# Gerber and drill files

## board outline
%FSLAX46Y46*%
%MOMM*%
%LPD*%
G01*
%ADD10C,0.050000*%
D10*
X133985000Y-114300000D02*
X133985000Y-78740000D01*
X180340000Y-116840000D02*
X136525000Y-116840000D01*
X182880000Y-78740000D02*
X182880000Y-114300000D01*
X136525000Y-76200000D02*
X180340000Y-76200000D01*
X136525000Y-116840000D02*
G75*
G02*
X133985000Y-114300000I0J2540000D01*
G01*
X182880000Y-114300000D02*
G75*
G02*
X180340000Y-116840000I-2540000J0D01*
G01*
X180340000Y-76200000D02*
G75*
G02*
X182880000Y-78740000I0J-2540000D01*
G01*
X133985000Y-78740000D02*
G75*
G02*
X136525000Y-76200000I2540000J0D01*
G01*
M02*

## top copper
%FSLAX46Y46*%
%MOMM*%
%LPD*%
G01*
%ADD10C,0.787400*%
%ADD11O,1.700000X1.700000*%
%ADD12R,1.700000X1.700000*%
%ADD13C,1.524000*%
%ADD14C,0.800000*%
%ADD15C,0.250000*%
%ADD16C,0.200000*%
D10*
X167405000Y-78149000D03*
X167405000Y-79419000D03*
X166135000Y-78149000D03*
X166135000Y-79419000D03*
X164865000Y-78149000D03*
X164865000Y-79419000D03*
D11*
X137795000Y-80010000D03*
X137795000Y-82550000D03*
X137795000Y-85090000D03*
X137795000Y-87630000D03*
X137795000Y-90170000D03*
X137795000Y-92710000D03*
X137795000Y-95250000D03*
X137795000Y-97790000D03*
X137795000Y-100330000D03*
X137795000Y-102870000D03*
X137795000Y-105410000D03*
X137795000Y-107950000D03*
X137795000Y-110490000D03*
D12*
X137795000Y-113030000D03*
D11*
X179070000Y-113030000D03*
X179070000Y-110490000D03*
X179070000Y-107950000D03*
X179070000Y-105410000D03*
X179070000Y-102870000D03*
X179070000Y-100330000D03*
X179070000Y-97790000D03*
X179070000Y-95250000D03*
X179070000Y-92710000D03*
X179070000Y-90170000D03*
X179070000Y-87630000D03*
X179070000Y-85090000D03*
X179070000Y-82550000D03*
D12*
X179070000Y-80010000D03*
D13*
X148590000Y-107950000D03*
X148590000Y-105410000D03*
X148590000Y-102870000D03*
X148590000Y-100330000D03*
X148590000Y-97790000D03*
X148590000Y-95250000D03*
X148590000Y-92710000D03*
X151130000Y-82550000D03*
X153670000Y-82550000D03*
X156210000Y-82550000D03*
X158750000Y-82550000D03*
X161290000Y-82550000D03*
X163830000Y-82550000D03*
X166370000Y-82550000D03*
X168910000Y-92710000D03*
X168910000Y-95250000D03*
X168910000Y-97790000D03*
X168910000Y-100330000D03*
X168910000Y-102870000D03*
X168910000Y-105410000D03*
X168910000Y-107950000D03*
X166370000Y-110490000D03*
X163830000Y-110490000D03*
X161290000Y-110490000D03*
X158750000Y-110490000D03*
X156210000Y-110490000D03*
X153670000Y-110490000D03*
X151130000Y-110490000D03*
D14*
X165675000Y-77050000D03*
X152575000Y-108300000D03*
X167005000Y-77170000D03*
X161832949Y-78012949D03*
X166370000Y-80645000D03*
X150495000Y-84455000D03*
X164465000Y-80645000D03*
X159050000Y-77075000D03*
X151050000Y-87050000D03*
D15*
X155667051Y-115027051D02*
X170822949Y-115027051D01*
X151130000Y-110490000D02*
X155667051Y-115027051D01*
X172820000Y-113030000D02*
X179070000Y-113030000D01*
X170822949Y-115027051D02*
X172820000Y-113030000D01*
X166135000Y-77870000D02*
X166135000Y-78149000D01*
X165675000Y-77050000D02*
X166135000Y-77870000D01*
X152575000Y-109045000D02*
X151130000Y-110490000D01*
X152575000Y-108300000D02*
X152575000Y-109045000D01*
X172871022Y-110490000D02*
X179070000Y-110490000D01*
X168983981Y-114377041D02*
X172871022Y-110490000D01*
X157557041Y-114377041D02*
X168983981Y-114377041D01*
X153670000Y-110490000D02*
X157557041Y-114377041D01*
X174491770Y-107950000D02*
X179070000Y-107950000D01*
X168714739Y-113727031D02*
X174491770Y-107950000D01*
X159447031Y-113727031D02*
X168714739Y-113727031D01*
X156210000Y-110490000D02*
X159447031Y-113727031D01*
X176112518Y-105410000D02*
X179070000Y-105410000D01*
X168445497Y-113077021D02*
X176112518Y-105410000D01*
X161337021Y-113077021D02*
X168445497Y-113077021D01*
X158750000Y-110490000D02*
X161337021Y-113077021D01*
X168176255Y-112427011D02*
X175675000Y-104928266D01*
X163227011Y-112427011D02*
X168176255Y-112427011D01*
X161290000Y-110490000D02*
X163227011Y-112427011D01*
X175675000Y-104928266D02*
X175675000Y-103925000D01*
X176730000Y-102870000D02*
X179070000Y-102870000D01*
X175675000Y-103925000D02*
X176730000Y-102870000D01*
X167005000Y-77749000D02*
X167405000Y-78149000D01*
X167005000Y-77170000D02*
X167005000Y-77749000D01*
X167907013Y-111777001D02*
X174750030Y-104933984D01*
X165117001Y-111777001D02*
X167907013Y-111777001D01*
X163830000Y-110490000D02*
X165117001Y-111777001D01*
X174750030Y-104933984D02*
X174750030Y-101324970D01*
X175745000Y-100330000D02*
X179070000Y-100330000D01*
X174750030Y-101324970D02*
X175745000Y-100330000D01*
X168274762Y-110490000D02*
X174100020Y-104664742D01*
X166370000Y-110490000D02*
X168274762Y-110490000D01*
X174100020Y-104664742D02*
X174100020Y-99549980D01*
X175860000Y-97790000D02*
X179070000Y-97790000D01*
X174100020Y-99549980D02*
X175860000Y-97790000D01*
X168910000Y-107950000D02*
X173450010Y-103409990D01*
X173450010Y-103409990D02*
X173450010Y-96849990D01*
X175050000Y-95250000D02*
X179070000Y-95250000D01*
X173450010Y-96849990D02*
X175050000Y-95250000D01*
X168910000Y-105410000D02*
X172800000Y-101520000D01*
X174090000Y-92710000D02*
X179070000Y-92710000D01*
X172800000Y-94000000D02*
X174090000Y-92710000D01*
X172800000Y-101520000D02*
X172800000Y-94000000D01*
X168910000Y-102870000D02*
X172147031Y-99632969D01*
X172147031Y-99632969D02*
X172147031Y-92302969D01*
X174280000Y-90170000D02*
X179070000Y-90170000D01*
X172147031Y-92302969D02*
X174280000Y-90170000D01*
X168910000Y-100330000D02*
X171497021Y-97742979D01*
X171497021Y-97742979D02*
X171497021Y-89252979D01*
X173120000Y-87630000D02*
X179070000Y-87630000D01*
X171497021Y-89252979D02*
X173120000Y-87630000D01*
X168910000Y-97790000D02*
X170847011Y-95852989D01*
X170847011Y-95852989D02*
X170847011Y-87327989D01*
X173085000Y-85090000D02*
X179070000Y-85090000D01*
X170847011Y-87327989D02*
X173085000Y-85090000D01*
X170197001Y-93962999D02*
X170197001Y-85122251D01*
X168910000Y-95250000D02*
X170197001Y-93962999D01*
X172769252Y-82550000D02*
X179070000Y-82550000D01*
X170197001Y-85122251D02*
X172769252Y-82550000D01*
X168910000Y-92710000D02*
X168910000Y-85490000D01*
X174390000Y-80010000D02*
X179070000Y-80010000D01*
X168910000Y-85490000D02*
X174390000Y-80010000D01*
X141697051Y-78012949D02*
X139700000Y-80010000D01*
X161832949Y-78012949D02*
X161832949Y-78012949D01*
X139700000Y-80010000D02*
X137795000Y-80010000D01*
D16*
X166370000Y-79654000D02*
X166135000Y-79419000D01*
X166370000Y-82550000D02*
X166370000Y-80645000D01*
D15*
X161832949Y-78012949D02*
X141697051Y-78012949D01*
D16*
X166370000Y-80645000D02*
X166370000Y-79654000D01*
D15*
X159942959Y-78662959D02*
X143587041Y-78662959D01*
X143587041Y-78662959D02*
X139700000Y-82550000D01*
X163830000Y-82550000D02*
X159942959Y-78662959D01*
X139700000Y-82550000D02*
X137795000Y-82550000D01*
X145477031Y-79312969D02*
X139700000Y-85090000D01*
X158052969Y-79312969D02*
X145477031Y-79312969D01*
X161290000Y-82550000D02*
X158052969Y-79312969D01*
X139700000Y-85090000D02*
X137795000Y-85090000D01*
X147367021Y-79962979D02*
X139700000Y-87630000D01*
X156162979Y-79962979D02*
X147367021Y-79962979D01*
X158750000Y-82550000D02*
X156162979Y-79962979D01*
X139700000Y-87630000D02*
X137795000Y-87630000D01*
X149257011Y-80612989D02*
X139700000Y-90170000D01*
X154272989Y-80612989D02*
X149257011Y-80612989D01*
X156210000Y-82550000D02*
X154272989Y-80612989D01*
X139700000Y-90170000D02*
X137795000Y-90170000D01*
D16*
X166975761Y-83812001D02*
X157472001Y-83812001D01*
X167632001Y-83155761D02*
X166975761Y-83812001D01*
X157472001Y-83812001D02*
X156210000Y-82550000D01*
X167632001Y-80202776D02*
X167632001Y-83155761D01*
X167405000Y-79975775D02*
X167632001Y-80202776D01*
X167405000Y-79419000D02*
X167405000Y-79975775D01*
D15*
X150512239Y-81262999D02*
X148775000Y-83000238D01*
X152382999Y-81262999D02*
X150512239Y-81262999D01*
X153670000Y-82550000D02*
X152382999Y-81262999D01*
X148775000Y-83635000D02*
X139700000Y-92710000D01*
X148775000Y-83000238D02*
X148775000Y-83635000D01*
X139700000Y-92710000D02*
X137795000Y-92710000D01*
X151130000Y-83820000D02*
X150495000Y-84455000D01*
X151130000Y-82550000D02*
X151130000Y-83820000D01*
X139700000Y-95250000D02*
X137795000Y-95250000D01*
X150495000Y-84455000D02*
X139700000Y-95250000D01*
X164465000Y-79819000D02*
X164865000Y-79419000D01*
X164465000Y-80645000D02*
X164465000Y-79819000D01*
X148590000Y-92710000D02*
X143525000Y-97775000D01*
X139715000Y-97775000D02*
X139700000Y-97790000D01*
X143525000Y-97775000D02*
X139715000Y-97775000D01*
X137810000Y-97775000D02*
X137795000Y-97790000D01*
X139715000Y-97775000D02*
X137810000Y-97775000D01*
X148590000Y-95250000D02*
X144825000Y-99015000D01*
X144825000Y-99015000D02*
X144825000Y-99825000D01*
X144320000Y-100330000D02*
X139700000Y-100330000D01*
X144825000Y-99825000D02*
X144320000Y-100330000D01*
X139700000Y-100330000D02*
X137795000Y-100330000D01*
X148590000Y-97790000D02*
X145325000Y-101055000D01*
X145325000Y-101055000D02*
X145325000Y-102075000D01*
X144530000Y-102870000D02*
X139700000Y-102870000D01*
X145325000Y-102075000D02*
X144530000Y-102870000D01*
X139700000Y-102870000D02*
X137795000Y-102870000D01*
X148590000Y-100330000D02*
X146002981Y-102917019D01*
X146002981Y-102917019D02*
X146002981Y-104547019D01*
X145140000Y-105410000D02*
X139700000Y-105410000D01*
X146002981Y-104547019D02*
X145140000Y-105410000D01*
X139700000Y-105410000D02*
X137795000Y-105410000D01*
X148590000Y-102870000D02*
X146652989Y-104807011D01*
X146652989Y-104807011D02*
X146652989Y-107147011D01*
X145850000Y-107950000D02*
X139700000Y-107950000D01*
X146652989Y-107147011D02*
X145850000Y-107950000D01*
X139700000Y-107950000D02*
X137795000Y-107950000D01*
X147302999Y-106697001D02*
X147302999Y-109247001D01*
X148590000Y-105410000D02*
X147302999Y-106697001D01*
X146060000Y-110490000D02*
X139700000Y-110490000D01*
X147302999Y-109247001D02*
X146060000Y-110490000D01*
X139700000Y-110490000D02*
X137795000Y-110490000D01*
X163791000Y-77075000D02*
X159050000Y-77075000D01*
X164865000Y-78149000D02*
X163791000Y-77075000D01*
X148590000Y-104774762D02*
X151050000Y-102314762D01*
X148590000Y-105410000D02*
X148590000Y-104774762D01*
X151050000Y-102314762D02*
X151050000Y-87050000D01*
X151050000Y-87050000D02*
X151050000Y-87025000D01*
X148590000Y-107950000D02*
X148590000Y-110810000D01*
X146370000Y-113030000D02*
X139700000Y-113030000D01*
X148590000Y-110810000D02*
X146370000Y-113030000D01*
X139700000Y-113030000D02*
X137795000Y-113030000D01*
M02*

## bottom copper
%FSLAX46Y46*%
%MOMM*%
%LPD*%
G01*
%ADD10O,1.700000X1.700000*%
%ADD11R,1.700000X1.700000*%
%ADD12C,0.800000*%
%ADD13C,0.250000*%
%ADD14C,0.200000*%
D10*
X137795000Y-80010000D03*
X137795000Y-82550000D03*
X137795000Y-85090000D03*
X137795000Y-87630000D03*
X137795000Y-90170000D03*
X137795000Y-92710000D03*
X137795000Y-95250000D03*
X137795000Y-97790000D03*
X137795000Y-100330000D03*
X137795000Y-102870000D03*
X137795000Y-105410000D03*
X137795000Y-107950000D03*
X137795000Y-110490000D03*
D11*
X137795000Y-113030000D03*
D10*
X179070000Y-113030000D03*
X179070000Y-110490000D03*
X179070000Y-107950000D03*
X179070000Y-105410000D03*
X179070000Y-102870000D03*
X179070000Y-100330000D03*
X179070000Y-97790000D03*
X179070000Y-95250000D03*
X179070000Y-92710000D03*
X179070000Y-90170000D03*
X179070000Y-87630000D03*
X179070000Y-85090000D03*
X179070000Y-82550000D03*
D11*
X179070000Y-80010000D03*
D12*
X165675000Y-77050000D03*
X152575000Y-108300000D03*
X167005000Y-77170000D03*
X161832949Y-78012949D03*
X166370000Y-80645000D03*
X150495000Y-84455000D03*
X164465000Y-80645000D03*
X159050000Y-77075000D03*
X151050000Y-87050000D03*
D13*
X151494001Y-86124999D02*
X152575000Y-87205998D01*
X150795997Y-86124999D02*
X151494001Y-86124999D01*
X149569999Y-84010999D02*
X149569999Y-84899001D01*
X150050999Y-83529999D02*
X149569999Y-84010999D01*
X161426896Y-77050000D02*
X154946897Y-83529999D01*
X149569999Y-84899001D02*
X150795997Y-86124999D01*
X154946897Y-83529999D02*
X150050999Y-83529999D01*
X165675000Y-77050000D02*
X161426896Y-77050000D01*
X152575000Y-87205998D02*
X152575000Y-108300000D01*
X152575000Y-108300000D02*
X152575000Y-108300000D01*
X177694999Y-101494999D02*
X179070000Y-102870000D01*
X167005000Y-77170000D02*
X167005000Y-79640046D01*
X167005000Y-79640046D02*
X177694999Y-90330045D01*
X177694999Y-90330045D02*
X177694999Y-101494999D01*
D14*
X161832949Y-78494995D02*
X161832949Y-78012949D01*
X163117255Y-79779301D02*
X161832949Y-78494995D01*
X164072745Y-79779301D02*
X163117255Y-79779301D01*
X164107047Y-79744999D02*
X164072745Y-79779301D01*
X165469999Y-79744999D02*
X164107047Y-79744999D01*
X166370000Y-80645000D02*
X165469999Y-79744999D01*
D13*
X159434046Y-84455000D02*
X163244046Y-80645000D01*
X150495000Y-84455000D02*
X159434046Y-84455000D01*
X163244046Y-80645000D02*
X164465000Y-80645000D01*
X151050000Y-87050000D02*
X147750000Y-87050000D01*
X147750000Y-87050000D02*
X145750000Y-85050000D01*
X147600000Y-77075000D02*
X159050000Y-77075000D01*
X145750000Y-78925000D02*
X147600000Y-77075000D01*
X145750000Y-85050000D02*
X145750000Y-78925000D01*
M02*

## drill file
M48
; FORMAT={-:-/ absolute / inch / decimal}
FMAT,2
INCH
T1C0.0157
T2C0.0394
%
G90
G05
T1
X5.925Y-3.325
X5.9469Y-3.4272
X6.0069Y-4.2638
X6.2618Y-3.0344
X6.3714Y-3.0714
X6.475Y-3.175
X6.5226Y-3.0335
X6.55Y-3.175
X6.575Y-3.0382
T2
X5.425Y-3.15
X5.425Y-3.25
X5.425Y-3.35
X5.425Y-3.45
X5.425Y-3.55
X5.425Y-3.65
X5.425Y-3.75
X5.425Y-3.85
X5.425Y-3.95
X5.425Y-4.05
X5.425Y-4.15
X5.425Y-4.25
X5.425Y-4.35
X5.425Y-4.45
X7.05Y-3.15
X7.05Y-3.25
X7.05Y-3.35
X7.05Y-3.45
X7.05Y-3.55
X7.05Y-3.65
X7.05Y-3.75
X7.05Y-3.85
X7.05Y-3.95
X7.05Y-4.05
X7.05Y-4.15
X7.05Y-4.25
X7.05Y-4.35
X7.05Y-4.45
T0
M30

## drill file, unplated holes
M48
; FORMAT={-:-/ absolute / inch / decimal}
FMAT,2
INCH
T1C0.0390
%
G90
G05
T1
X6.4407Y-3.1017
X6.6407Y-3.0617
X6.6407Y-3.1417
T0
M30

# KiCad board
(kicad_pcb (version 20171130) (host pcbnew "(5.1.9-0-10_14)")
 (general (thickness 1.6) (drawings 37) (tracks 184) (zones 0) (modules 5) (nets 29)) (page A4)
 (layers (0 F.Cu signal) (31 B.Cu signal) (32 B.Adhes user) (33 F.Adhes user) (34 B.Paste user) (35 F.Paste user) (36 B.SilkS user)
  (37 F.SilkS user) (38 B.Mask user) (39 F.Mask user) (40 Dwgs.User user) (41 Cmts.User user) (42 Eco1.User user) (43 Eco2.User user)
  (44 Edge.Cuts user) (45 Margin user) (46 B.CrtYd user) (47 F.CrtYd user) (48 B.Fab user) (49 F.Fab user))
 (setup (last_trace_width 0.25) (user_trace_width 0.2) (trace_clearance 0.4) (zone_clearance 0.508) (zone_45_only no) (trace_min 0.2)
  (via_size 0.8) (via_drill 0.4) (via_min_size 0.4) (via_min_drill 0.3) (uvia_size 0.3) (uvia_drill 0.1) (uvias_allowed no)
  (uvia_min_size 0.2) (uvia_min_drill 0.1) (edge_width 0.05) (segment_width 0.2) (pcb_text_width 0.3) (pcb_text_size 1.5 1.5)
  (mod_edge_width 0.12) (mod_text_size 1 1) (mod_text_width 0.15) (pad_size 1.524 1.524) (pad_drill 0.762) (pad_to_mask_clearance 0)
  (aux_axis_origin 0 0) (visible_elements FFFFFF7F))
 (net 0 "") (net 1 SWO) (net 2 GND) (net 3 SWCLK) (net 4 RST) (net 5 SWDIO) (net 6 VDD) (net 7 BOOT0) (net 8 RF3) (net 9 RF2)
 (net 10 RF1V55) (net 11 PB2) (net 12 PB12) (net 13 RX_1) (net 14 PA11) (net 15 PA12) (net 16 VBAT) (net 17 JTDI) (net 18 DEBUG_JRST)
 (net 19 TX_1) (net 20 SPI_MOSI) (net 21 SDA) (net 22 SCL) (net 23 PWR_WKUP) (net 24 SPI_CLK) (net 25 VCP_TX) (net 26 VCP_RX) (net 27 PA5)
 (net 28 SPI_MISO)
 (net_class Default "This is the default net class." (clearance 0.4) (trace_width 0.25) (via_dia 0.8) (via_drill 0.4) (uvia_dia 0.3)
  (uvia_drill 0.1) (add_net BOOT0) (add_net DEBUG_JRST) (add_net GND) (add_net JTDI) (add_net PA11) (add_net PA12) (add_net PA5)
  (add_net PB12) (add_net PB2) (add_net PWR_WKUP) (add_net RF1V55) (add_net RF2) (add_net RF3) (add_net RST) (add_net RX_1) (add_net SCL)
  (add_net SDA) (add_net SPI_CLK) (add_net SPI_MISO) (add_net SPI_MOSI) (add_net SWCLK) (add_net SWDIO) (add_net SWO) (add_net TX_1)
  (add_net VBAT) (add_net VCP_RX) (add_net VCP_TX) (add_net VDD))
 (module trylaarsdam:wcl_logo (layer F.Cu) (at 148 114.25)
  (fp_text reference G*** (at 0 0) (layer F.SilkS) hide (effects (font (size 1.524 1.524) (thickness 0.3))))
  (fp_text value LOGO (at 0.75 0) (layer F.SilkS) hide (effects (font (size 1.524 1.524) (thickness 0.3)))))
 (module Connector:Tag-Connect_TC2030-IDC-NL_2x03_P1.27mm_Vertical (layer F.Cu) (at 166.135 78.784)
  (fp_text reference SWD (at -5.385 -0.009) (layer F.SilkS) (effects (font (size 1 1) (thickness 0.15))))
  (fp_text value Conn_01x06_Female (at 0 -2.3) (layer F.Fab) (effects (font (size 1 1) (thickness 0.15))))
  (pad 6 connect circle (at 1.27 -0.635) (size 0.7874 0.7874) (layers F.Cu F.Mask) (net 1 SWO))
  (pad 5 connect circle (at 1.27 0.635) (size 0.7874 0.7874) (layers F.Cu F.Mask) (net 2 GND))
  (pad 4 connect circle (at 0 -0.635) (size 0.7874 0.7874) (layers F.Cu F.Mask) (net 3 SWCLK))
  (pad 3 connect circle (at 0 0.635) (size 0.7874 0.7874) (layers F.Cu F.Mask) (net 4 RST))
  (pad 2 connect circle (at -1.27 -0.635) (size 0.7874 0.7874) (layers F.Cu F.Mask) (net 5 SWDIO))
  (pad 1 connect circle (at -1.27 0.635) (size 0.7874 0.7874) (layers F.Cu F.Mask) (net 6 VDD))
  (pad "" np_thru_hole circle (at -2.54 0) (size 0.9906 0.9906) (drill 0.9906) (layers *.Cu *.Mask))
  (pad "" np_thru_hole circle (at 2.54 1.016) (size 0.9906 0.9906) (drill 0.9906) (layers *.Cu *.Mask))
  (pad "" np_thru_hole circle (at 2.54 -1.016) (size 0.9906 0.9906) (drill 0.9906) (layers *.Cu *.Mask)))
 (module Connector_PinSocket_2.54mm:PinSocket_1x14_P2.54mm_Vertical (layer F.Cu) (at 137.795 113.03 180)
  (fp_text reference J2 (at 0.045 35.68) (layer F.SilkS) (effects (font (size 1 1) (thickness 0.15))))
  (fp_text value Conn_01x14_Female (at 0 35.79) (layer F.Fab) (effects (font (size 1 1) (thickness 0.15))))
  (pad 14 thru_hole oval (at 0 33.02 180) (size 1.7 1.7) (drill 1) (layers *.Cu *.Mask) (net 4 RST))
  (pad 13 thru_hole oval (at 0 30.48 180) (size 1.7 1.7) (drill 1) (layers *.Cu *.Mask) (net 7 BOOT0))
  (pad 12 thru_hole oval (at 0 27.94 180) (size 1.7 1.7) (drill 1) (layers *.Cu *.Mask) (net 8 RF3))
  (pad 11 thru_hole oval (at 0 25.4 180) (size 1.7 1.7) (drill 1) (layers *.Cu *.Mask) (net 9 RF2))
  (pad 10 thru_hole oval (at 0 22.86 180) (size 1.7 1.7) (drill 1) (layers *.Cu *.Mask) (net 2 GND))
  (pad 9 thru_hole oval (at 0 20.32 180) (size 1.7 1.7) (drill 1) (layers *.Cu *.Mask) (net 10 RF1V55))
  (pad 8 thru_hole oval (at 0 17.78 180) (size 1.7 1.7) (drill 1) (layers *.Cu *.Mask) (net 6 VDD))
  (pad 7 thru_hole oval (at 0 15.24 180) (size 1.7 1.7) (drill 1) (layers *.Cu *.Mask) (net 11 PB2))
  (pad 6 thru_hole oval (at 0 12.7 180) (size 1.7 1.7) (drill 1) (layers *.Cu *.Mask) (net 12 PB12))
  (pad 5 thru_hole oval (at 0 10.16 180) (size 1.7 1.7) (drill 1) (layers *.Cu *.Mask) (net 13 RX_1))
  (pad 4 thru_hole oval (at 0 7.62 180) (size 1.7 1.7) (drill 1) (layers *.Cu *.Mask) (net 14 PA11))
  (pad 3 thru_hole oval (at 0 5.08 180) (size 1.7 1.7) (drill 1) (layers *.Cu *.Mask) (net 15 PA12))
  (pad 2 thru_hole oval (at 0 2.54 180) (size 1.7 1.7) (drill 1) (layers *.Cu *.Mask) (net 5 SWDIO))
  (pad 1 thru_hole rect (at 0 0 180) (size 1.7 1.7) (drill 1) (layers *.Cu *.Mask) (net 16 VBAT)))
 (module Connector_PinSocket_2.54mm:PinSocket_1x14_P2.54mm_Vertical (layer F.Cu) (at 179.07 80.01)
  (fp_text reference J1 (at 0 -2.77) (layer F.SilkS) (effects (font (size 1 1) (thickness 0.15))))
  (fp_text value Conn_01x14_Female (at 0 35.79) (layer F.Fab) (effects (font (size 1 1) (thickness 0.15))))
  (pad 14 thru_hole oval (at 0 33.02) (size 1.7 1.7) (drill 1) (layers *.Cu *.Mask) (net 3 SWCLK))
  (pad 13 thru_hole oval (at 0 30.48) (size 1.7 1.7) (drill 1) (layers *.Cu *.Mask) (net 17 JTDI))
  (pad 12 thru_hole oval (at 0 27.94) (size 1.7 1.7) (drill 1) (layers *.Cu *.Mask) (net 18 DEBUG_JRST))
  (pad 11 thru_hole oval (at 0 25.4) (size 1.7 1.7) (drill 1) (layers *.Cu *.Mask) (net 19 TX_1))
  (pad 10 thru_hole oval (at 0 22.86) (size 1.7 1.7) (drill 1) (layers *.Cu *.Mask) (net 1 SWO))
  (pad 9 thru_hole oval (at 0 20.32) (size 1.7 1.7) (drill 1) (layers *.Cu *.Mask) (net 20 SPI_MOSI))
  (pad 8 thru_hole oval (at 0 17.78) (size 1.7 1.7) (drill 1) (layers *.Cu *.Mask) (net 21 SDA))
  (pad 7 thru_hole oval (at 0 15.24) (size 1.7 1.7) (drill 1) (layers *.Cu *.Mask) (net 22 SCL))
  (pad 6 thru_hole oval (at 0 12.7) (size 1.7 1.7) (drill 1) (layers *.Cu *.Mask) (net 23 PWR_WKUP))
  (pad 5 thru_hole oval (at 0 10.16) (size 1.7 1.7) (drill 1) (layers *.Cu *.Mask) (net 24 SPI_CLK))
  (pad 4 thru_hole oval (at 0 7.62) (size 1.7 1.7) (drill 1) (layers *.Cu *.Mask) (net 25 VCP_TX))
  (pad 3 thru_hole oval (at 0 5.08) (size 1.7 1.7) (drill 1) (layers *.Cu *.Mask) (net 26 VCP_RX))
  (pad 2 thru_hole oval (at 0 2.54) (size 1.7 1.7) (drill 1) (layers *.Cu *.Mask) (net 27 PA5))
  (pad 1 thru_hole rect (at 0 0) (size 1.7 1.7) (drill 1) (layers *.Cu *.Mask) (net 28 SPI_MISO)))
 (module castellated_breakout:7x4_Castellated (layer F.Cu) (at 163.83 97.79 90)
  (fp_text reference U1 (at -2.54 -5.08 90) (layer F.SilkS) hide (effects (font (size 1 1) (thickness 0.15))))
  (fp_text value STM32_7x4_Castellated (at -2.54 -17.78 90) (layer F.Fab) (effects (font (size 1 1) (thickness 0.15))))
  (pad 28 smd circle (at -10.16 -15.24 90) (size 1.524 1.524) (layers F.Cu F.Paste F.Mask) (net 16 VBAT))
  (pad 27 smd circle (at -7.62 -15.24 90) (size 1.524 1.524) (layers F.Cu F.Paste F.Mask) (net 5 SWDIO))
  (pad 26 smd circle (at -5.08 -15.24 90) (size 1.524 1.524) (layers F.Cu F.Paste F.Mask) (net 15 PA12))
  (pad 25 smd circle (at -2.54 -15.24 90) (size 1.524 1.524) (layers F.Cu F.Paste F.Mask) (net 14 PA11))
  (pad 24 smd circle (at 0 -15.24 90) (size 1.524 1.524) (layers F.Cu F.Paste F.Mask) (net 13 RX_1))
  (pad 23 smd circle (at 2.54 -15.24 90) (size 1.524 1.524) (layers F.Cu F.Paste F.Mask) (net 12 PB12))
  (pad 22 smd circle (at 5.08 -15.24 90) (size 1.524 1.524) (layers F.Cu F.Paste F.Mask) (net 11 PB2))
  (pad 21 smd circle (at 15.24 -12.7 90) (size 1.524 1.524) (layers F.Cu F.Paste F.Mask) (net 6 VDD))
  (pad 20 smd circle (at 15.24 -10.16 90) (size 1.524 1.524) (layers F.Cu F.Paste F.Mask) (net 10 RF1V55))
  (pad 19 smd circle (at 15.24 -7.62 90) (size 1.524 1.524) (layers F.Cu F.Paste F.Mask) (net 2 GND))
  (pad 18 smd circle (at 15.24 -5.08 90) (size 1.524 1.524) (layers F.Cu F.Paste F.Mask) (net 9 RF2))
  (pad 17 smd circle (at 15.24 -2.54 90) (size 1.524 1.524) (layers F.Cu F.Paste F.Mask) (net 8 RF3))
  (pad 16 smd circle (at 15.24 0 90) (size 1.524 1.524) (layers F.Cu F.Paste F.Mask) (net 7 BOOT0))
  (pad 15 smd circle (at 15.24 2.54 90) (size 1.524 1.524) (layers F.Cu F.Paste F.Mask) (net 4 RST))
  (pad 14 smd circle (at 5.08 5.08 90) (size 1.524 1.524) (layers F.Cu F.Paste F.Mask) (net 28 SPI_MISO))
  (pad 13 smd circle (at 2.54 5.08 90) (size 1.524 1.524) (layers F.Cu F.Paste F.Mask) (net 27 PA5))
  (pad 12 smd circle (at 0 5.08 90) (size 1.524 1.524) (layers F.Cu F.Paste F.Mask) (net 26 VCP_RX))
  (pad 11 smd circle (at -2.54 5.08 90) (size 1.524 1.524) (layers F.Cu F.Paste F.Mask) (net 25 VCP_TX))
  (pad 10 smd circle (at -5.08 5.08 90) (size 1.524 1.524) (layers F.Cu F.Paste F.Mask) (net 24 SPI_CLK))
  (pad 9 smd circle (at -7.62 5.08 90) (size 1.524 1.524) (layers F.Cu F.Paste F.Mask) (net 23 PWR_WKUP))
  (pad 8 smd circle (at -10.16 5.08 90) (size 1.524 1.524) (layers F.Cu F.Paste F.Mask) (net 22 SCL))
  (pad 7 smd circle (at -12.7 2.54 90) (size 1.524 1.524) (layers F.Cu F.Paste F.Mask) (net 21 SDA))
  (pad 6 smd circle (at -12.7 0 90) (size 1.524 1.524) (layers F.Cu F.Paste F.Mask) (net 20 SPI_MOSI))
  (pad 5 smd circle (at -12.7 -2.54 90) (size 1.524 1.524) (layers F.Cu F.Paste F.Mask) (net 1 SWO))
  (pad 4 smd circle (at -12.7 -5.08 90) (size 1.524 1.524) (layers F.Cu F.Paste F.Mask) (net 19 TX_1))
  (pad 3 smd circle (at -12.7 -7.62 90) (size 1.524 1.524) (layers F.Cu F.Paste F.Mask) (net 18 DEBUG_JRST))
  (pad 2 smd circle (at -12.7 -10.16 90) (size 1.524 1.524) (layers F.Cu F.Paste F.Mask) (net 17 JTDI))
  (pad 1 smd circle (at -12.7 -12.7 90) (size 1.524 1.524) (layers F.Cu F.Paste F.Mask) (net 3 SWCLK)))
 (gr_line (start 133.985 114.3) (end 133.985 78.74) (layer Edge.Cuts) (width 0.05))
 (gr_line (start 180.34 116.84) (end 136.525 116.84) (layer Edge.Cuts) (width 0.05))
 (gr_line (start 182.88 78.74) (end 182.88 114.3) (layer Edge.Cuts) (width 0.05))
 (gr_line (start 136.525 76.2) (end 180.34 76.2) (layer Edge.Cuts) (width 0.05))
 (gr_arc (start 136.525 114.3) (end 133.985 114.3) (angle -90) (layer Edge.Cuts) (width 0.05))
 (gr_arc (start 180.34 114.3) (end 180.34 116.84) (angle -90) (layer Edge.Cuts) (width 0.05))
 (gr_arc (start 180.34 78.74) (end 182.88 78.74) (angle -90) (layer Edge.Cuts) (width 0.05))
 (gr_arc (start 136.525 78.74) (end 136.525 76.2) (angle -90) (layer Edge.Cuts) (width 0.05))
 (segment (start 155.667051 115.027051) (end 170.822949 115.027051) (width 0.25) (layer F.Cu) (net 3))
 (segment (start 151.13 110.49) (end 155.667051 115.027051) (width 0.25) (layer F.Cu) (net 3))
 (segment (start 172.82 113.03) (end 179.07 113.03) (width 0.25) (layer F.Cu) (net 3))
 (segment (start 170.822949 115.027051) (end 172.82 113.03) (width 0.25) (layer F.Cu) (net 3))
 (segment (start 166.135 77.87) (end 166.135 78.149) (width 0.25) (layer F.Cu) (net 3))
 (segment (start 165.675 77.05) (end 166.135 77.87) (width 0.25) (layer F.Cu) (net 3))
 (via (at 165.675 77.05) (size 0.8) (drill 0.4) (layers F.Cu B.Cu) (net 3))
 (segment (start 151.494001 86.124999) (end 152.575 87.205998) (width 0.25) (layer B.Cu) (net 3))
 (segment (start 150.795997 86.124999) (end 151.494001 86.124999) (width 0.25) (layer B.Cu) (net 3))
 (segment (start 149.569999 84.010999) (end 149.569999 84.899001) (width 0.25) (layer B.Cu) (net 3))
 (segment (start 150.050999 83.529999) (end 149.569999 84.010999) (width 0.25) (layer B.Cu) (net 3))
 (segment (start 161.426896 77.05) (end 154.946897 83.529999) (width 0.25) (layer B.Cu) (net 3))
 (segment (start 149.569999 84.899001) (end 150.795997 86.124999) (width 0.25) (layer B.Cu) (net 3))
 (segment (start 154.946897 83.529999) (end 150.050999 83.529999) (width 0.25) (layer B.Cu) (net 3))
 (segment (start 165.675 77.05) (end 161.426896 77.05) (width 0.25) (layer B.Cu) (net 3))
 (segment (start 152.575 87.205998) (end 152.575 108.3) (width 0.25) (layer B.Cu) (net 3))
 (segment (start 152.575 108.3) (end 152.575 108.3) (width 0.25) (layer B.Cu) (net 3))
 (via (at 152.575 108.3) (size 0.8) (drill 0.4) (layers F.Cu B.Cu) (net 3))
 (segment (start 152.575 109.045) (end 151.13 110.49) (width 0.25) (layer F.Cu) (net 3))
 (segment (start 152.575 108.3) (end 152.575 109.045) (width 0.25) (layer F.Cu) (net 3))
 (segment (start 172.871022 110.49) (end 179.07 110.49) (width 0.25) (layer F.Cu) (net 17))
 (segment (start 168.983981 114.377041) (end 172.871022 110.49) (width 0.25) (layer F.Cu) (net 17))
 (segment (start 157.557041 114.377041) (end 168.983981 114.377041) (width 0.25) (layer F.Cu) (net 17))
 (segment (start 153.67 110.49) (end 157.557041 114.377041) (width 0.25) (layer F.Cu) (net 17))
 (segment (start 174.49177 107.95) (end 179.07 107.95) (width 0.25) (layer F.Cu) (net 18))
 (segment (start 168.714739 113.727031) (end 174.49177 107.95) (width 0.25) (layer F.Cu) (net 18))
 (segment (start 159.447031 113.727031) (end 168.714739 113.727031) (width 0.25) (layer F.Cu) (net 18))
 (segment (start 156.21 110.49) (end 159.447031 113.727031) (width 0.25) (layer F.Cu) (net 18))
 (segment (start 176.112518 105.41) (end 179.07 105.41) (width 0.25) (layer F.Cu) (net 19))
 (segment (start 168.445497 113.077021) (end 176.112518 105.41) (width 0.25) (layer F.Cu) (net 19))
 (segment (start 161.337021 113.077021) (end 168.445497 113.077021) (width 0.25) (layer F.Cu) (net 19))
 (segment (start 158.75 110.49) (end 161.337021 113.077021) (width 0.25) (layer F.Cu) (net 19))
 (segment (start 168.176255 112.427011) (end 175.675 104.928266) (width 0.25) (layer F.Cu) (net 1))
 (segment (start 163.227011 112.427011) (end 168.176255 112.427011) (width 0.25) (layer F.Cu) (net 1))
 (segment (start 161.29 110.49) (end 163.227011 112.427011) (width 0.25) (layer F.Cu) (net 1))
 (segment (start 175.675 104.928266) (end 175.675 103.925) (width 0.25) (layer F.Cu) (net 1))
 (segment (start 176.73 102.87) (end 179.07 102.87) (width 0.25) (layer F.Cu) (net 1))
 (segment (start 175.675 103.925) (end 176.73 102.87) (width 0.25) (layer F.Cu) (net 1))
 (segment (start 177.694999 101.494999) (end 179.07 102.87) (width 0.25) (layer B.Cu) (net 1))
 (segment (start 167.005 77.17) (end 167.005 79.640046) (width 0.25) (layer B.Cu) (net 1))
 (segment (start 167.005 77.749) (end 167.405 78.149) (width 0.25) (layer F.Cu) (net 1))
 (segment (start 167.005 79.640046) (end 177.694999 90.330045) (width 0.25) (layer B.Cu) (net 1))
 (segment (start 177.694999 90.330045) (end 177.694999 101.494999) (width 0.25) (layer B.Cu) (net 1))
 (segment (start 167.005 77.17) (end 167.005 77.749) (width 0.25) (layer F.Cu) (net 1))
 (via (at 167.005 77.17) (size 0.8) (drill 0.4) (layers F.Cu B.Cu) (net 1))
 (segment (start 167.907013 111.777001) (end 174.75003 104.933984) (width 0.25) (layer F.Cu) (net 20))
 (segment (start 165.117001 111.777001) (end 167.907013 111.777001) (width 0.25) (layer F.Cu) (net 20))
 (segment (start 163.83 110.49) (end 165.117001 111.777001) (width 0.25) (layer F.Cu) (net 20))
 (segment (start 174.75003 104.933984) (end 174.75003 101.32497) (width 0.25) (layer F.Cu) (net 20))
 (segment (start 175.745 100.33) (end 179.07 100.33) (width 0.25) (layer F.Cu) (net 20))
 (segment (start 174.75003 101.32497) (end 175.745 100.33) (width 0.25) (layer F.Cu) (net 20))
 (segment (start 168.274762 110.49) (end 174.10002 104.664742) (width 0.25) (layer F.Cu) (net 21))
 (segment (start 166.37 110.49) (end 168.274762 110.49) (width 0.25) (layer F.Cu) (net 21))
 (segment (start 174.10002 104.664742) (end 174.10002 99.54998) (width 0.25) (layer F.Cu) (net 21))
 (segment (start 175.86 97.79) (end 179.07 97.79) (width 0.25) (layer F.Cu) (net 21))
 (segment (start 174.10002 99.54998) (end 175.86 97.79) (width 0.25) (layer F.Cu) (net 21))
 (segment (start 168.91 107.95) (end 173.45001 103.40999) (width 0.25) (layer F.Cu) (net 22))
 (segment (start 173.45001 103.40999) (end 173.45001 96.84999) (width 0.25) (layer F.Cu) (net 22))
 (segment (start 175.05 95.25) (end 179.07 95.25) (width 0.25) (layer F.Cu) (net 22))
 (segment (start 173.45001 96.84999) (end 175.05 95.25) (width 0.25) (layer F.Cu) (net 22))
 (segment (start 168.91 105.41) (end 172.8 101.52) (width 0.25) (layer F.Cu) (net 23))
 (segment (start 174.09 92.71) (end 179.07 92.71) (width 0.25) (layer F.Cu) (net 23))
 (segment (start 172.8 94) (end 174.09 92.71) (width 0.25) (layer F.Cu) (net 23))
 (segment (start 172.8 101.52) (end 172.8 94) (width 0.25) (layer F.Cu) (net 23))
 (segment (start 168.91 102.87) (end 172.147031 99.632969) (width 0.25) (layer F.Cu) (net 24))
 (segment (start 172.147031 99.632969) (end 172.147031 92.302969) (width 0.25) (layer F.Cu) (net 24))
 (segment (start 174.28 90.17) (end 179.07 90.17) (width 0.25) (layer F.Cu) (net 24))
 (segment (start 172.147031 92.302969) (end 174.28 90.17) (width 0.25) (layer F.Cu) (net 24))
 (segment (start 168.91 100.33) (end 171.497021 97.742979) (width 0.25) (layer F.Cu) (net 25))
 (segment (start 171.497021 97.742979) (end 171.497021 89.252979) (width 0.25) (layer F.Cu) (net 25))
 (segment (start 173.12 87.63) (end 179.07 87.63) (width 0.25) (layer F.Cu) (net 25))
 (segment (start 171.497021 89.252979) (end 173.12 87.63) (width 0.25) (layer F.Cu) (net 25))
 (segment (start 168.91 97.79) (end 170.847011 95.852989) (width 0.25) (layer F.Cu) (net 26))
 (segment (start 170.847011 95.852989) (end 170.847011 87.327989) (width 0.25) (layer F.Cu) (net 26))
 (segment (start 173.085 85.09) (end 179.07 85.09) (width 0.25) (layer F.Cu) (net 26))
 (segment (start 170.847011 87.327989) (end 173.085 85.09) (width 0.25) (layer F.Cu) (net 26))
 (segment (start 170.197001 93.962999) (end 170.197001 85.122251) (width 0.25) (layer F.Cu) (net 27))
 (segment (start 168.91 95.25) (end 170.197001 93.962999) (width 0.25) (layer F.Cu) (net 27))
 (segment (start 172.769252 82.55) (end 179.07 82.55) (width 0.25) (layer F.Cu) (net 27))
 (segment (start 170.197001 85.122251) (end 172.769252 82.55) (width 0.25) (layer F.Cu) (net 27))
 (segment (start 168.91 92.71) (end 168.91 85.49) (width 0.25) (layer F.Cu) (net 28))
 (segment (start 174.39 80.01) (end 179.07 80.01) (width 0.25) (layer F.Cu) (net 28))
 (segment (start 168.91 85.49) (end 174.39 80.01) (width 0.25) (layer F.Cu) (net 28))
 (segment (start 141.697051 78.012949) (end 139.7 80.01) (width 0.25) (layer F.Cu) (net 4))
 (segment (start 161.832949 78.012949) (end 161.832949 78.012949) (width 0.25) (layer F.Cu) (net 4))
 (segment (start 139.7 80.01) (end 137.795 80.01) (width 0.25) (layer F.Cu) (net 4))
 (segment (start 166.37 79.654) (end 166.135 79.419) (width 0.2) (layer F.Cu) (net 4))
 (segment (start 166.37 82.55) (end 166.37 80.645) (width 0.2) (layer F.Cu) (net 4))
 (segment (start 161.832949 78.012949) (end 141.697051 78.012949) (width 0.25) (layer F.Cu) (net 4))
 (via (at 161.832949 78.012949) (size 0.8) (drill 0.4) (layers F.Cu B.Cu) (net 4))
 (segment (start 166.37 80.645) (end 166.37 79.654) (width 0.2) (layer F.Cu) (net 4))
 (via (at 166.37 80.645) (size 0.8) (drill 0.4) (layers F.Cu B.Cu) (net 4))
 (segment (start 161.832949 78.494995) (end 161.832949 78.012949) (width 0.2) (layer B.Cu) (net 4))
 (segment (start 163.117255 79.779301) (end 161.832949 78.494995) (width 0.2) (layer B.Cu) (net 4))
 (segment (start 164.072745 79.779301) (end 163.117255 79.779301) (width 0.2) (layer B.Cu) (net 4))
 (segment (start 164.107047 79.744999) (end 164.072745 79.779301) (width 0.2) (layer B.Cu) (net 4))
 (segment (start 165.469999 79.744999) (end 164.107047 79.744999) (width 0.2) (layer B.Cu) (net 4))
 (segment (start 166.37 80.645) (end 165.469999 79.744999) (width 0.2) (layer B.Cu) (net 4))
 (segment (start 159.942959 78.662959) (end 143.587041 78.662959) (width 0.25) (layer F.Cu) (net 7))
 (segment (start 143.587041 78.662959) (end 139.7 82.55) (width 0.25) (layer F.Cu) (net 7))
 (segment (start 163.83 82.55) (end 159.942959 78.662959) (width 0.25) (layer F.Cu) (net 7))
 (segment (start 139.7 82.55) (end 137.795 82.55) (width 0.25) (layer F.Cu) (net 7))
 (segment (start 145.477031 79.312969) (end 139.7 85.09) (width 0.25) (layer F.Cu) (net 8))
 (segment (start 158.052969 79.312969) (end 145.477031 79.312969) (width 0.25) (layer F.Cu) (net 8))
 (segment (start 161.29 82.55) (end 158.052969 79.312969) (width 0.25) (layer F.Cu) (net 8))
 (segment (start 139.7 85.09) (end 137.795 85.09) (width 0.25) (layer F.Cu) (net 8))
 (segment (start 147.367021 79.962979) (end 139.7 87.63) (width 0.25) (layer F.Cu) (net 9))
 (segment (start 156.162979 79.962979) (end 147.367021 79.962979) (width 0.25) (layer F.Cu) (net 9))
 (segment (start 158.75 82.55) (end 156.162979 79.962979) (width 0.25) (layer F.Cu) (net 9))
 (segment (start 139.7 87.63) (end 137.795 87.63) (width 0.25) (layer F.Cu) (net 9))
 (segment (start 149.257011 80.612989) (end 139.7 90.17) (width 0.25) (layer F.Cu) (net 2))
 (segment (start 154.272989 80.612989) (end 149.257011 80.612989) (width 0.25) (layer F.Cu) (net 2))
 (segment (start 156.21 82.55) (end 154.272989 80.612989) (width 0.25) (layer F.Cu) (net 2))
 (segment (start 139.7 90.17) (end 137.795 90.17) (width 0.25) (layer F.Cu) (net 2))
 (segment (start 166.975761 83.812001) (end 157.472001 83.812001) (width 0.2) (layer F.Cu) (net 2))
 (segment (start 167.632001 83.155761) (end 166.975761 83.812001) (width 0.2) (layer F.Cu) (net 2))
 (segment (start 157.472001 83.812001) (end 156.21 82.55) (width 0.2) (layer F.Cu) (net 2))
 (segment (start 167.632001 80.202776) (end 167.632001 83.155761) (width 0.2) (layer F.Cu) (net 2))
 (segment (start 167.405 79.975775) (end 167.632001 80.202776) (width 0.2) (layer F.Cu) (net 2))
 (segment (start 167.405 79.419) (end 167.405 79.975775) (width 0.2) (layer F.Cu) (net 2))
 (segment (start 150.512239 81.262999) (end 148.775 83.000238) (width 0.25) (layer F.Cu) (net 10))
 (segment (start 152.382999 81.262999) (end 150.512239 81.262999) (width 0.25) (layer F.Cu) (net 10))
 (segment (start 153.67 82.55) (end 152.382999 81.262999) (width 0.25) (layer F.Cu) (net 10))
 (segment (start 148.775 83.635) (end 139.7 92.71) (width 0.25) (layer F.Cu) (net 10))
 (segment (start 148.775 83.000238) (end 148.775 83.635) (width 0.25) (layer F.Cu) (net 10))
 (segment (start 139.7 92.71) (end 137.795 92.71) (width 0.25) (layer F.Cu) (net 10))
 (segment (start 151.13 83.82) (end 150.495 84.455) (width 0.25) (layer F.Cu) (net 6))
 (segment (start 151.13 82.55) (end 151.13 83.82) (width 0.25) (layer F.Cu) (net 6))
 (segment (start 139.7 95.25) (end 137.795 95.25) (width 0.25) (layer F.Cu) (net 6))
 (segment (start 150.495 84.455) (end 139.7 95.25) (width 0.25) (layer F.Cu) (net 6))
 (via (at 150.495 84.455) (size 0.8) (drill 0.4) (layers F.Cu B.Cu) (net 6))
 (segment (start 159.434046 84.455) (end 163.244046 80.645) (width 0.25) (layer B.Cu) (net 6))
 (segment (start 150.495 84.455) (end 159.434046 84.455) (width 0.25) (layer B.Cu) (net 6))
 (segment (start 163.244046 80.645) (end 164.465 80.645) (width 0.25) (layer B.Cu) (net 6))
 (via (at 164.465 80.645) (size 0.8) (drill 0.4) (layers F.Cu B.Cu) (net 6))
 (segment (start 164.465 79.819) (end 164.865 79.419) (width 0.25) (layer F.Cu) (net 6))
 (segment (start 164.465 80.645) (end 164.465 79.819) (width 0.25) (layer F.Cu) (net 6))
 (segment (start 148.59 92.71) (end 143.525 97.775) (width 0.25) (layer F.Cu) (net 11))
 (segment (start 139.715 97.775) (end 139.7 97.79) (width 0.25) (layer F.Cu) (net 11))
 (segment (start 143.525 97.775) (end 139.715 97.775) (width 0.25) (layer F.Cu) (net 11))
 (segment (start 137.81 97.775) (end 137.795 97.79) (width 0.25) (layer F.Cu) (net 11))
 (segment (start 139.715 97.775) (end 137.81 97.775) (width 0.25) (layer F.Cu) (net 11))
 (segment (start 148.59 95.25) (end 144.825 99.015) (width 0.25) (layer F.Cu) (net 12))
 (segment (start 144.825 99.015) (end 144.825 99.825) (width 0.25) (layer F.Cu) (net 12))
 (segment (start 144.32 100.33) (end 139.7 100.33) (width 0.25) (layer F.Cu) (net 12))
 (segment (start 144.825 99.825) (end 144.32 100.33) (width 0.25) (layer F.Cu) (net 12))
 (segment (start 139.7 100.33) (end 137.795 100.33) (width 0.25) (layer F.Cu) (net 12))
 (segment (start 148.59 97.79) (end 145.325 101.055) (width 0.25) (layer F.Cu) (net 13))
 (segment (start 145.325 101.055) (end 145.325 102.075) (width 0.25) (layer F.Cu) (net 13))
 (segment (start 144.53 102.87) (end 139.7 102.87) (width 0.25) (layer F.Cu) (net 13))
 (segment (start 145.325 102.075) (end 144.53 102.87) (width 0.25) (layer F.Cu) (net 13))
 (segment (start 139.7 102.87) (end 137.795 102.87) (width 0.25) (layer F.Cu) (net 13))
 (segment (start 148.59 100.33) (end 146.002981 102.917019) (width 0.25) (layer F.Cu) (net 14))
 (segment (start 146.002981 102.917019) (end 146.002981 104.547019) (width 0.25) (layer F.Cu) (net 14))
 (segment (start 145.14 105.41) (end 139.7 105.41) (width 0.25) (layer F.Cu) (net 14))
 (segment (start 146.002981 104.547019) (end 145.14 105.41) (width 0.25) (layer F.Cu) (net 14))
 (segment (start 139.7 105.41) (end 137.795 105.41) (width 0.25) (layer F.Cu) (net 14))
 (segment (start 148.59 102.87) (end 146.652989 104.807011) (width 0.25) (layer F.Cu) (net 15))
 (segment (start 146.652989 104.807011) (end 146.652989 107.147011) (width 0.25) (layer F.Cu) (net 15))
 (segment (start 145.85 107.95) (end 139.7 107.95) (width 0.25) (layer F.Cu) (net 15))
 (segment (start 146.652989 107.147011) (end 145.85 107.95) (width 0.25) (layer F.Cu) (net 15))
 (segment (start 139.7 107.95) (end 137.795 107.95) (width 0.25) (layer F.Cu) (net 15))
 (segment (start 147.302999 106.697001) (end 147.302999 109.247001) (width 0.25) (layer F.Cu) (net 5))
 (segment (start 148.59 105.41) (end 147.302999 106.697001) (width 0.25) (layer F.Cu) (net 5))
 (segment (start 146.06 110.49) (end 139.7 110.49) (width 0.25) (layer F.Cu) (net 5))
 (segment (start 147.302999 109.247001) (end 146.06 110.49) (width 0.25) (layer F.Cu) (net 5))
 (segment (start 139.7 110.49) (end 137.795 110.49) (width 0.25) (layer F.Cu) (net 5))
 (via (at 159.05 77.075) (size 0.8) (drill 0.4) (layers F.Cu B.Cu) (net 5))
 (segment (start 163.791 77.075) (end 159.05 77.075) (width 0.25) (layer F.Cu) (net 5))
 (segment (start 164.865 78.149) (end 163.791 77.075) (width 0.25) (layer F.Cu) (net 5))
 (segment (start 148.59 104.774762) (end 151.05 102.314762) (width 0.25) (layer F.Cu) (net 5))
 (segment (start 148.59 105.41) (end 148.59 104.774762) (width 0.25) (layer F.Cu) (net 5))
 (segment (start 151.05 102.314762) (end 151.05 87.05) (width 0.25) (layer F.Cu) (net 5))
 (segment (start 151.05 87.05) (end 151.05 87.025) (width 0.25) (layer F.Cu) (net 5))
 (via (at 151.05 87.05) (size 0.8) (drill 0.4) (layers F.Cu B.Cu) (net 5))
 (segment (start 151.05 87.05) (end 147.75 87.05) (width 0.25) (layer B.Cu) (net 5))
 (segment (start 147.75 87.05) (end 145.75 85.05) (width 0.25) (layer B.Cu) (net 5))
 (segment (start 147.6 77.075) (end 159.05 77.075) (width 0.25) (layer B.Cu) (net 5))
 (segment (start 145.75 78.925) (end 147.6 77.075) (width 0.25) (layer B.Cu) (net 5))
 (segment (start 145.75 85.05) (end 145.75 78.925) (width 0.25) (layer B.Cu) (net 5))
 (segment (start 148.59 107.95) (end 148.59 110.81) (width 0.25) (layer F.Cu) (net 16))
 (segment (start 146.37 113.03) (end 139.7 113.03) (width 0.25) (layer F.Cu) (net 16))
 (segment (start 148.59 110.81) (end 146.37 113.03) (width 0.25) (layer F.Cu) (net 16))
 (segment (start 139.7 113.03) (end 137.795 113.03) (width 0.25) (layer F.Cu) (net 16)))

